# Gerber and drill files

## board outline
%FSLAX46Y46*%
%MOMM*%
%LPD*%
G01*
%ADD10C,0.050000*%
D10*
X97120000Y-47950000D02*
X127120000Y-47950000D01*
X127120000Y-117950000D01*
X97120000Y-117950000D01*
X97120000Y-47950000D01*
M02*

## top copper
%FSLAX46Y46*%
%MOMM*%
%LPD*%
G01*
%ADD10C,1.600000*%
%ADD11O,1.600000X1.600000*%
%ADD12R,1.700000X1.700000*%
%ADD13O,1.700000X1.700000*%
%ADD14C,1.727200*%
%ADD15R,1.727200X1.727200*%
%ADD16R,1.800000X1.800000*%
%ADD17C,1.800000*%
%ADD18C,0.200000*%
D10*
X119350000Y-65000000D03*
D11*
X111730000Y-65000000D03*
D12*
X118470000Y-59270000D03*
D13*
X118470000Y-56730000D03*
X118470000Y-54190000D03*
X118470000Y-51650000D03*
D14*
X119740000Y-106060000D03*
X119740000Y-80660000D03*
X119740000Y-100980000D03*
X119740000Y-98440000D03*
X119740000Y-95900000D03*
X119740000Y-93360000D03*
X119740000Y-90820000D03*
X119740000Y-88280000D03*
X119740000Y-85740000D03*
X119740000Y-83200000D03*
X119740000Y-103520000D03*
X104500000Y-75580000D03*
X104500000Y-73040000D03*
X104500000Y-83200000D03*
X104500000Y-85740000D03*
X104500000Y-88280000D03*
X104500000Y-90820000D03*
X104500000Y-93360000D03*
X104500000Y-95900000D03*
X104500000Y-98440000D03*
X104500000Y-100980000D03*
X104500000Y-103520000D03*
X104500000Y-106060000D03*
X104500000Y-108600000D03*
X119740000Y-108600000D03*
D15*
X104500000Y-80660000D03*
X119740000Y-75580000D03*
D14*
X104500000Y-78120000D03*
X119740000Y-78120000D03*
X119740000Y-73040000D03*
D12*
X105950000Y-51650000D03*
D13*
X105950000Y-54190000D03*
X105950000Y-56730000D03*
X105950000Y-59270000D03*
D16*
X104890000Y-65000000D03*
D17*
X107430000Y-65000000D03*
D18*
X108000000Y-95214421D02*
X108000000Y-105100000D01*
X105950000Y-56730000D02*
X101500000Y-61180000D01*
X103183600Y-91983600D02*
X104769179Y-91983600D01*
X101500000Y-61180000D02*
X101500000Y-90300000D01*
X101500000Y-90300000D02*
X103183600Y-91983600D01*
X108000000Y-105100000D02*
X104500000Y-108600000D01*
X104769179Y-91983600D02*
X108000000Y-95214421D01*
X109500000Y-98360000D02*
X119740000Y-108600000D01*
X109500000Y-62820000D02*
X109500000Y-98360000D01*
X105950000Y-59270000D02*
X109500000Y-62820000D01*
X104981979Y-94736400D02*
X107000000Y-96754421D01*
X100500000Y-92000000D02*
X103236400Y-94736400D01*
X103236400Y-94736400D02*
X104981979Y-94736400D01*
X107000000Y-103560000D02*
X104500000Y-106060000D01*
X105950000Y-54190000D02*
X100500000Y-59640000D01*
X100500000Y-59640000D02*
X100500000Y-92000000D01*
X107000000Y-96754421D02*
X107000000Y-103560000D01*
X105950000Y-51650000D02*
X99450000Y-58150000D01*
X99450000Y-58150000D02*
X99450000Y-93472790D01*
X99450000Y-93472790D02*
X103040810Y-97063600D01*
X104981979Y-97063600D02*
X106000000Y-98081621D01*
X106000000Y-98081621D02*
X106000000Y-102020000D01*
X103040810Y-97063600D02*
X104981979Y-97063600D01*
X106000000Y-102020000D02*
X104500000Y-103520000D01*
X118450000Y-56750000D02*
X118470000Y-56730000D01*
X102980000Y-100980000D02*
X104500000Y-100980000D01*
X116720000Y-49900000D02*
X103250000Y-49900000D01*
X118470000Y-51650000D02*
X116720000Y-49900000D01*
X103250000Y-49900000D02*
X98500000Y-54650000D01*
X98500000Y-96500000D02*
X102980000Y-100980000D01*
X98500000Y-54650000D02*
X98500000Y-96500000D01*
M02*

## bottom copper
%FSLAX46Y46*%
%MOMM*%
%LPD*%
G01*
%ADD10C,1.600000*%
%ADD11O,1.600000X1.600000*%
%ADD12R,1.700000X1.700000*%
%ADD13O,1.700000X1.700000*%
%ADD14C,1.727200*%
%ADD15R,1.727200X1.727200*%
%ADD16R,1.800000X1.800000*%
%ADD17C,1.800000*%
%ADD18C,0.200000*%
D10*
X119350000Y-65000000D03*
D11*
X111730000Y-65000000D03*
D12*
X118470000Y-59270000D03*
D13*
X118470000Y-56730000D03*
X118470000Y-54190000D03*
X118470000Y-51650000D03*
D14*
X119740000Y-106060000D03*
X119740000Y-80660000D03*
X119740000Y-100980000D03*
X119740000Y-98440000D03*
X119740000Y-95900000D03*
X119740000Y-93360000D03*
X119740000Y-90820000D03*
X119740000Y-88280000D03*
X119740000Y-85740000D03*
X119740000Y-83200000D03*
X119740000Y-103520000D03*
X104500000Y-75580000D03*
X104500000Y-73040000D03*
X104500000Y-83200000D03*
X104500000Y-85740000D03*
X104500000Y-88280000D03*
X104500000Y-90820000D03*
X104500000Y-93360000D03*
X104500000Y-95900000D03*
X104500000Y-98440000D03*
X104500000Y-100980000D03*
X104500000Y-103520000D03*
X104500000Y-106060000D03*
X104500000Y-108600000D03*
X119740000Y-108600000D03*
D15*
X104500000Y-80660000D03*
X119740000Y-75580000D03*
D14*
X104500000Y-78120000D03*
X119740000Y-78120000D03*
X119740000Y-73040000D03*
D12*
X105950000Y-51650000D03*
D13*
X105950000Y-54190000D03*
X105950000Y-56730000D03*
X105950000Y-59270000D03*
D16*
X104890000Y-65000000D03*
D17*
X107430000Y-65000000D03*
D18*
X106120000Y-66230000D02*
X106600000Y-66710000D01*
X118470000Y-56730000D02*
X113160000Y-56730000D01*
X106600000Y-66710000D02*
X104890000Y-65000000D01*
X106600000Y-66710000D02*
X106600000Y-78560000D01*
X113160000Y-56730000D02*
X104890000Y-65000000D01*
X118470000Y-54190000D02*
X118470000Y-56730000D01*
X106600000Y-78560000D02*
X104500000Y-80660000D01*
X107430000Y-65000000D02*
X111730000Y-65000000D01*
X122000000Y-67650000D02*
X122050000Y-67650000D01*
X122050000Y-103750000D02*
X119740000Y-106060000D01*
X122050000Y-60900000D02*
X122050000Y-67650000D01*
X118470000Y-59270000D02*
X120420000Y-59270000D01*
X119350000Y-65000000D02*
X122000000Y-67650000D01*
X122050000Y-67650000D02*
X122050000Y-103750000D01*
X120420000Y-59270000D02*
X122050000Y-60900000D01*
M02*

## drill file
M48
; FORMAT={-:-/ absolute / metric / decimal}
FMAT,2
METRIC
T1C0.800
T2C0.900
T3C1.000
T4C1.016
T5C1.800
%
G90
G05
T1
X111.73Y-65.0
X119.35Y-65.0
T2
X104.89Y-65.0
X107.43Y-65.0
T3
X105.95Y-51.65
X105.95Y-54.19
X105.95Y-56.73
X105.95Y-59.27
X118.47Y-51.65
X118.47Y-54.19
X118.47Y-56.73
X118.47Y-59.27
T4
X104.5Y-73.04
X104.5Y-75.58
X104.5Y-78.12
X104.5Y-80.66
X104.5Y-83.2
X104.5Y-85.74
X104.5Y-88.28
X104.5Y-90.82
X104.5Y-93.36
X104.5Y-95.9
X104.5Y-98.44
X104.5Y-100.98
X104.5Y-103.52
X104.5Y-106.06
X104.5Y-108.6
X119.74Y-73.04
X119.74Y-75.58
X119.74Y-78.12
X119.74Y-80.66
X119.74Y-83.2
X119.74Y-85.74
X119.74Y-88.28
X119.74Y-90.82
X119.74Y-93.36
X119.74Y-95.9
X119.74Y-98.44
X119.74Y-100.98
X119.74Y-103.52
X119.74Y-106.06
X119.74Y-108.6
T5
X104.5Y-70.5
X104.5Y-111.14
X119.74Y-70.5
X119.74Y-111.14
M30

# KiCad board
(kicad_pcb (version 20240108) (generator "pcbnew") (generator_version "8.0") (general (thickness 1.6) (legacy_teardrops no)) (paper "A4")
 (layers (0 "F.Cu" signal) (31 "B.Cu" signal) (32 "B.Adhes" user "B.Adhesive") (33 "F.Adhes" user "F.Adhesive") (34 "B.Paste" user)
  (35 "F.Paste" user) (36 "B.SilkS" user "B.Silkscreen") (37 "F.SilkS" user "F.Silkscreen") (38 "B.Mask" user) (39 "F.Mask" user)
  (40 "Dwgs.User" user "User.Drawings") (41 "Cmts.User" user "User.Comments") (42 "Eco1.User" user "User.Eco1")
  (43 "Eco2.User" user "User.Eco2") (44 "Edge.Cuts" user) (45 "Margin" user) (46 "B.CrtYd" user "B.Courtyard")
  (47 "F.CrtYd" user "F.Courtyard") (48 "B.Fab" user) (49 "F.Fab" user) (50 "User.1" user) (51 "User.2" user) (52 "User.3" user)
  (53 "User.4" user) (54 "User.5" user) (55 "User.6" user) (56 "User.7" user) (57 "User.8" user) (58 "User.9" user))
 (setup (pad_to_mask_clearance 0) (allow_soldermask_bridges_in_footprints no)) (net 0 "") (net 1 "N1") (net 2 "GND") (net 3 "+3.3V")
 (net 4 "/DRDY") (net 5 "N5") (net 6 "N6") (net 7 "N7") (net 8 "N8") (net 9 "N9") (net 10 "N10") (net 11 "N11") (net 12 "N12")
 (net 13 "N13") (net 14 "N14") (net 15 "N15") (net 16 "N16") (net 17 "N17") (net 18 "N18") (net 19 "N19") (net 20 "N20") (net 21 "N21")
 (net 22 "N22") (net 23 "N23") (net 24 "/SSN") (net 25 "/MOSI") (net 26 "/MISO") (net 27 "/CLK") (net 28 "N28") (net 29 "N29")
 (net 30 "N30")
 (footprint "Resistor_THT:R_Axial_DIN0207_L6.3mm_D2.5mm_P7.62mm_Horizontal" (layer "F.Cu") (at 119.35 65 180)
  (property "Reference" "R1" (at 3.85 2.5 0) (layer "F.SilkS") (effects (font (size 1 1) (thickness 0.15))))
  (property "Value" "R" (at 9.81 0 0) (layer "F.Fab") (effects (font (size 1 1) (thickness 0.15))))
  (pad "1" thru_hole circle (at 0 0 180) (size 1.6 1.6) (drill 0.8) (layers "*.Cu" "*.Mask") (remove_unused_layers no) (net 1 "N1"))
  (pad "2" thru_hole oval (at 7.62 0 180) (size 1.6 1.6) (drill 0.8) (layers "*.Cu" "*.Mask") (remove_unused_layers no) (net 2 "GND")))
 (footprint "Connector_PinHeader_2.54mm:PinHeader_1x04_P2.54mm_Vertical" (layer "F.Cu") (at 118.47 59.27 180)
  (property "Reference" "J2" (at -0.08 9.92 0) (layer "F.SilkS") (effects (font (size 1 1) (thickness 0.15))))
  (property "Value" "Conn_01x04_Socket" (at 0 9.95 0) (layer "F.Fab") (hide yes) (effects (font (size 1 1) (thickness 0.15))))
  (pad "1" thru_hole rect (at 0 0 180) (size 1.7 1.7) (drill 1) (layers "*.Cu" "*.Mask") (remove_unused_layers no) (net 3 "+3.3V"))
  (pad "2" thru_hole oval (at 0 2.54 180) (size 1.7 1.7) (drill 1) (layers "*.Cu" "*.Mask") (remove_unused_layers no) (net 2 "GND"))
  (pad "3" thru_hole oval (at 0 5.08 180) (size 1.7 1.7) (drill 1) (layers "*.Cu" "*.Mask") (remove_unused_layers no) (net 2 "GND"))
  (pad "4" thru_hole oval (at 0 7.62 180) (size 1.7 1.7) (drill 1) (layers "*.Cu" "*.Mask") (remove_unused_layers no) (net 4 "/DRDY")))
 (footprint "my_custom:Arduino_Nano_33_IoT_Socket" (layer "F.Cu") (at 112.12 112.41)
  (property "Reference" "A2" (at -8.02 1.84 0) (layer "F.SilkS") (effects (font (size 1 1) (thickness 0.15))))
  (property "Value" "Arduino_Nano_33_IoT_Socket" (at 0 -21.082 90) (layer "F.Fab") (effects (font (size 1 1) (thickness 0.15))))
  (pad "" np_thru_hole circle (at -7.62 -41.91) (size 1.8 1.8) (drill 1.8) (layers "F&B.Cu" "*.Mask"))
  (pad "" np_thru_hole circle (at -7.62 -1.27) (size 1.8 1.8) (drill 1.8) (layers "F&B.Cu" "*.Mask"))
  (pad "" np_thru_hole circle (at 7.62 -41.91) (size 1.8 1.8) (drill 1.8) (layers "F&B.Cu" "*.Mask"))
  (pad "" np_thru_hole circle (at 7.62 -1.27) (size 1.8 1.8) (drill 1.8) (layers "F&B.Cu" "*.Mask"))
  (pad "3V3" thru_hole circle (at 7.62 -6.35) (size 1.7272 1.7272) (drill 1.016) (layers "*.Cu" "*.Mask") (remove_unused_layers no)
   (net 3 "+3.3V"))
  (pad "5V" thru_hole circle (at 7.62 -31.75) (size 1.7272 1.7272) (drill 1.016) (layers "*.Cu" "*.Mask") (remove_unused_layers no)
   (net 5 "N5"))
  (pad "A0" thru_hole circle (at 7.62 -11.43) (size 1.7272 1.7272) (drill 1.016) (layers "*.Cu" "*.Mask") (remove_unused_layers no)
   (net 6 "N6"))
  (pad "A1" thru_hole circle (at 7.62 -13.97) (size 1.7272 1.7272) (drill 1.016) (layers "*.Cu" "*.Mask") (remove_unused_layers no)
   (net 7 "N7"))
  (pad "A2" thru_hole circle (at 7.62 -16.51) (size 1.7272 1.7272) (drill 1.016) (layers "*.Cu" "*.Mask") (remove_unused_layers no)
   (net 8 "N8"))
  (pad "A3" thru_hole circle (at 7.62 -19.05) (size 1.7272 1.7272) (drill 1.016) (layers "*.Cu" "*.Mask") (remove_unused_layers no)
   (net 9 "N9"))
  (pad "A4" thru_hole circle (at 7.62 -21.59) (size 1.7272 1.7272) (drill 1.016) (layers "*.Cu" "*.Mask") (remove_unused_layers no)
   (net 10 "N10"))
  (pad "A5" thru_hole circle (at 7.62 -24.13) (size 1.7272 1.7272) (drill 1.016) (layers "*.Cu" "*.Mask") (remove_unused_layers no)
   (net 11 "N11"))
  (pad "A6" thru_hole circle (at 7.62 -26.67) (size 1.7272 1.7272) (drill 1.016) (layers "*.Cu" "*.Mask") (remove_unused_layers no)
   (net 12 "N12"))
  (pad "A7" thru_hole circle (at 7.62 -29.21) (size 1.7272 1.7272) (drill 1.016) (layers "*.Cu" "*.Mask") (remove_unused_layers no)
   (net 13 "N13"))
  (pad "AREF" thru_hole circle (at 7.62 -8.89) (size 1.7272 1.7272) (drill 1.016) (layers "*.Cu" "*.Mask") (remove_unused_layers no)
   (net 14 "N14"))
  (pad "D0" thru_hole circle (at -7.62 -36.83) (size 1.7272 1.7272) (drill 1.016) (layers "*.Cu" "*.Mask") (remove_unused_layers no)
   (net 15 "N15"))
  (pad "D1" thru_hole circle (at -7.62 -39.37) (size 1.7272 1.7272) (drill 1.016) (layers "*.Cu" "*.Mask") (remove_unused_layers no)
   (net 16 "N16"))
  (pad "D2" thru_hole circle (at -7.62 -29.21) (size 1.7272 1.7272) (drill 1.016) (layers "*.Cu" "*.Mask") (remove_unused_layers no)
   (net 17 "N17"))
  (pad "D3" thru_hole circle (at -7.62 -26.67) (size 1.7272 1.7272) (drill 1.016) (layers "*.Cu" "*.Mask") (remove_unused_layers no)
   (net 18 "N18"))
  (pad "D4" thru_hole circle (at -7.62 -24.13) (size 1.7272 1.7272) (drill 1.016) (layers "*.Cu" "*.Mask") (remove_unused_layers no)
   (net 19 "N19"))
  (pad "D5" thru_hole circle (at -7.62 -21.59) (size 1.7272 1.7272) (drill 1.016) (layers "*.Cu" "*.Mask") (remove_unused_layers no)
   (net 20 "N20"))
  (pad "D6" thru_hole circle (at -7.62 -19.05) (size 1.7272 1.7272) (drill 1.016) (layers "*.Cu" "*.Mask") (remove_unused_layers no)
   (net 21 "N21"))
  (pad "D7" thru_hole circle (at -7.62 -16.51) (size 1.7272 1.7272) (drill 1.016) (layers "*.Cu" "*.Mask") (remove_unused_layers no)
   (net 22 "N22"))
  (pad "D8" thru_hole circle (at -7.62 -13.97) (size 1.7272 1.7272) (drill 1.016) (layers "*.Cu" "*.Mask") (remove_unused_layers no)
   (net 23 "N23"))
  (pad "D9" thru_hole circle (at -7.62 -11.43) (size 1.7272 1.7272) (drill 1.016) (layers "*.Cu" "*.Mask") (remove_unused_layers no)
   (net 4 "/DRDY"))
  (pad "D10" thru_hole circle (at -7.62 -8.89) (size 1.7272 1.7272) (drill 1.016) (layers "*.Cu" "*.Mask") (remove_unused_layers no)
   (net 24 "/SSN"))
  (pad "D11" thru_hole circle (at -7.62 -6.35) (size 1.7272 1.7272) (drill 1.016) (layers "*.Cu" "*.Mask") (remove_unused_layers no)
   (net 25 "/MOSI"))
  (pad "D12" thru_hole circle (at -7.62 -3.81) (size 1.7272 1.7272) (drill 1.016) (layers "*.Cu" "*.Mask") (remove_unused_layers no)
   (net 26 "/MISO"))
  (pad "D13" thru_hole circle (at 7.62 -3.81) (size 1.7272 1.7272) (drill 1.016) (layers "*.Cu" "*.Mask") (remove_unused_layers no)
   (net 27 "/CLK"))
  (pad "GND" thru_hole rect (at -7.62 -31.75) (size 1.7272 1.7272) (drill 1.016) (layers "*.Cu" "*.Mask") (remove_unused_layers no))
  (pad "GND" thru_hole rect (at 7.62 -36.83) (size 1.7272 1.7272) (drill 1.016) (layers "*.Cu" "*.Mask") (remove_unused_layers no))
  (pad "RST1" thru_hole circle (at -7.62 -34.29) (size 1.7272 1.7272) (drill 1.016) (layers "*.Cu" "*.Mask") (remove_unused_layers no)
   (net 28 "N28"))
  (pad "RST2" thru_hole circle (at 7.62 -34.29) (size 1.7272 1.7272) (drill 1.016) (layers "*.Cu" "*.Mask") (remove_unused_layers no)
   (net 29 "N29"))
  (pad "VIN" thru_hole circle (at 7.62 -39.37) (size 1.7272 1.7272) (drill 1.016) (layers "*.Cu" "*.Mask") (remove_unused_layers no)
   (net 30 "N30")))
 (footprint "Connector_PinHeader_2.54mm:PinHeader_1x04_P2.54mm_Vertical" (layer "F.Cu") (at 105.95 51.65)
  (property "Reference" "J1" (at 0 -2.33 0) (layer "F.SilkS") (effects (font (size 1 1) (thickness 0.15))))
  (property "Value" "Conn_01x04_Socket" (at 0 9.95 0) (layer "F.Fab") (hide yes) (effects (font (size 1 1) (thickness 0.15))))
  (pad "1" thru_hole rect (at 0 0) (size 1.7 1.7) (drill 1) (layers "*.Cu" "*.Mask") (remove_unused_layers no) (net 24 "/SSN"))
  (pad "2" thru_hole oval (at 0 2.54) (size 1.7 1.7) (drill 1) (layers "*.Cu" "*.Mask") (remove_unused_layers no) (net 25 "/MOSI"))
  (pad "3" thru_hole oval (at 0 5.08) (size 1.7 1.7) (drill 1) (layers "*.Cu" "*.Mask") (remove_unused_layers no) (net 26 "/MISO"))
  (pad "4" thru_hole oval (at 0 7.62) (size 1.7 1.7) (drill 1) (layers "*.Cu" "*.Mask") (remove_unused_layers no) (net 27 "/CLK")))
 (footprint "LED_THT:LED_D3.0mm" (layer "F.Cu") (at 104.89 65)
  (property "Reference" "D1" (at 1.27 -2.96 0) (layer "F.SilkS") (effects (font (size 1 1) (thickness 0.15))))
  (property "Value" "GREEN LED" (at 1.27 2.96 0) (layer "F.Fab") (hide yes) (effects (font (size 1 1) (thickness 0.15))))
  (pad "1" thru_hole rect (at 0 0) (size 1.8 1.8) (drill 0.9) (layers "*.Cu" "*.Mask") (remove_unused_layers no) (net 1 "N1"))
  (pad "2" thru_hole circle (at 2.54 0) (size 1.8 1.8) (drill 0.9) (layers "*.Cu" "*.Mask") (remove_unused_layers no) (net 3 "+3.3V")))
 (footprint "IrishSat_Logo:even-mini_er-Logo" (layer "F.Cu") (at 123.3 54.2)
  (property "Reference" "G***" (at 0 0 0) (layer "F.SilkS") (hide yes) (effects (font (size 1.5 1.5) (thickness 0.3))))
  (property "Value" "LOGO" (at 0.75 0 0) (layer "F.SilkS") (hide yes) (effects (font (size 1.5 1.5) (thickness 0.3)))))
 (gr_rect (start 97.12 47.95) (end 127.12 117.95) (locked yes) (stroke (width 0.05) (type solid)) (fill none) (layer "Edge.Cuts"))
 (segment (start 108 95.214421) (end 108 105.1) (width 0.2) (layer "F.Cu") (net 26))
 (segment (start 105.95 56.73) (end 101.5 61.18) (width 0.2) (layer "F.Cu") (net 26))
 (segment (start 103.1836 91.9836) (end 104.769179 91.9836) (width 0.2) (layer "F.Cu") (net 26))
 (segment (start 101.5 61.18) (end 101.5 90.3) (width 0.2) (layer "F.Cu") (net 26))
 (segment (start 101.5 90.3) (end 103.1836 91.9836) (width 0.2) (layer "F.Cu") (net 26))
 (segment (start 108 105.1) (end 104.5 108.6) (width 0.2) (layer "F.Cu") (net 26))
 (segment (start 104.769179 91.9836) (end 108 95.214421) (width 0.2) (layer "F.Cu") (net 26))
 (segment (start 109.5 98.36) (end 119.74 108.6) (width 0.2) (layer "F.Cu") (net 27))
 (segment (start 109.5 62.82) (end 109.5 98.36) (width 0.2) (layer "F.Cu") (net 27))
 (segment (start 105.95 59.27) (end 109.5 62.82) (width 0.2) (layer "F.Cu") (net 27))
 (segment (start 104.981979 94.7364) (end 107 96.754421) (width 0.2) (layer "F.Cu") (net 25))
 (segment (start 100.5 92) (end 103.2364 94.7364) (width 0.2) (layer "F.Cu") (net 25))
 (segment (start 103.2364 94.7364) (end 104.981979 94.7364) (width 0.2) (layer "F.Cu") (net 25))
 (segment (start 107 103.56) (end 104.5 106.06) (width 0.2) (layer "F.Cu") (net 25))
 (segment (start 105.95 54.19) (end 100.5 59.64) (width 0.2) (layer "F.Cu") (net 25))
 (segment (start 100.5 59.64) (end 100.5 92) (width 0.2) (layer "F.Cu") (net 25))
 (segment (start 107 96.754421) (end 107 103.56) (width 0.2) (layer "F.Cu") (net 25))
 (segment (start 105.95 51.65) (end 99.45 58.15) (width 0.2) (layer "F.Cu") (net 24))
 (segment (start 99.45 58.15) (end 99.45 93.47279) (width 0.2) (layer "F.Cu") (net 24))
 (segment (start 99.45 93.47279) (end 103.04081 97.0636) (width 0.2) (layer "F.Cu") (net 24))
 (segment (start 104.981979 97.0636) (end 106 98.081621) (width 0.2) (layer "F.Cu") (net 24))
 (segment (start 106 98.081621) (end 106 102.02) (width 0.2) (layer "F.Cu") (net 24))
 (segment (start 103.04081 97.0636) (end 104.981979 97.0636) (width 0.2) (layer "F.Cu") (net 24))
 (segment (start 106 102.02) (end 104.5 103.52) (width 0.2) (layer "F.Cu") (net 24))
 (segment (start 118.45 56.75) (end 118.47 56.73) (width 0.2) (layer "F.Cu") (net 2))
 (segment (start 106.12 66.23) (end 106.6 66.71) (width 0.2) (layer "B.Cu") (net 2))
 (segment (start 118.47 56.73) (end 113.16 56.73) (width 0.2) (layer "B.Cu") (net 2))
 (segment (start 106.6 66.71) (end 104.89 65) (width 0.2) (layer "B.Cu") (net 2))
 (segment (start 106.6 66.71) (end 106.6 78.56) (width 0.2) (layer "B.Cu") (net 2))
 (segment (start 113.16 56.73) (end 104.89 65) (width 0.2) (layer "B.Cu") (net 2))
 (segment (start 118.47 54.19) (end 118.47 56.73) (width 0.2) (layer "B.Cu") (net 2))
 (segment (start 106.6 78.56) (end 104.5 80.66) (width 0.2) (layer "B.Cu") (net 2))
 (segment (start 107.43 65) (end 111.73 65) (width 0.2) (layer "B.Cu") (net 3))
 (segment (start 122 67.65) (end 122.05 67.65) (width 0.2) (layer "B.Cu") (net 3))
 (segment (start 122.05 103.75) (end 119.74 106.06) (width 0.2) (layer "B.Cu") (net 3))
 (segment (start 122.05 60.9) (end 122.05 67.65) (width 0.2) (layer "B.Cu") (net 3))
 (segment (start 118.47 59.27) (end 120.42 59.27) (width 0.2) (layer "B.Cu") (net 3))
 (segment (start 119.35 65) (end 122 67.65) (width 0.2) (layer "B.Cu") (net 3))
 (segment (start 122.05 67.65) (end 122.05 103.75) (width 0.2) (layer "B.Cu") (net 3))
 (segment (start 120.42 59.27) (end 122.05 60.9) (width 0.2) (layer "B.Cu") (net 3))
 (segment (start 102.98 100.98) (end 104.5 100.98) (width 0.2) (layer "F.Cu") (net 4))
 (segment (start 116.72 49.9) (end 103.25 49.9) (width 0.2) (layer "F.Cu") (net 4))
 (segment (start 118.47 51.65) (end 116.72 49.9) (width 0.2) (layer "F.Cu") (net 4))
 (segment (start 103.25 49.9) (end 98.5 54.65) (width 0.2) (layer "F.Cu") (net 4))
 (segment (start 98.5 96.5) (end 102.98 100.98) (width 0.2) (layer "F.Cu") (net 4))
 (segment (start 98.5 54.65) (end 98.5 96.5) (width 0.2) (layer "F.Cu") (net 4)))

